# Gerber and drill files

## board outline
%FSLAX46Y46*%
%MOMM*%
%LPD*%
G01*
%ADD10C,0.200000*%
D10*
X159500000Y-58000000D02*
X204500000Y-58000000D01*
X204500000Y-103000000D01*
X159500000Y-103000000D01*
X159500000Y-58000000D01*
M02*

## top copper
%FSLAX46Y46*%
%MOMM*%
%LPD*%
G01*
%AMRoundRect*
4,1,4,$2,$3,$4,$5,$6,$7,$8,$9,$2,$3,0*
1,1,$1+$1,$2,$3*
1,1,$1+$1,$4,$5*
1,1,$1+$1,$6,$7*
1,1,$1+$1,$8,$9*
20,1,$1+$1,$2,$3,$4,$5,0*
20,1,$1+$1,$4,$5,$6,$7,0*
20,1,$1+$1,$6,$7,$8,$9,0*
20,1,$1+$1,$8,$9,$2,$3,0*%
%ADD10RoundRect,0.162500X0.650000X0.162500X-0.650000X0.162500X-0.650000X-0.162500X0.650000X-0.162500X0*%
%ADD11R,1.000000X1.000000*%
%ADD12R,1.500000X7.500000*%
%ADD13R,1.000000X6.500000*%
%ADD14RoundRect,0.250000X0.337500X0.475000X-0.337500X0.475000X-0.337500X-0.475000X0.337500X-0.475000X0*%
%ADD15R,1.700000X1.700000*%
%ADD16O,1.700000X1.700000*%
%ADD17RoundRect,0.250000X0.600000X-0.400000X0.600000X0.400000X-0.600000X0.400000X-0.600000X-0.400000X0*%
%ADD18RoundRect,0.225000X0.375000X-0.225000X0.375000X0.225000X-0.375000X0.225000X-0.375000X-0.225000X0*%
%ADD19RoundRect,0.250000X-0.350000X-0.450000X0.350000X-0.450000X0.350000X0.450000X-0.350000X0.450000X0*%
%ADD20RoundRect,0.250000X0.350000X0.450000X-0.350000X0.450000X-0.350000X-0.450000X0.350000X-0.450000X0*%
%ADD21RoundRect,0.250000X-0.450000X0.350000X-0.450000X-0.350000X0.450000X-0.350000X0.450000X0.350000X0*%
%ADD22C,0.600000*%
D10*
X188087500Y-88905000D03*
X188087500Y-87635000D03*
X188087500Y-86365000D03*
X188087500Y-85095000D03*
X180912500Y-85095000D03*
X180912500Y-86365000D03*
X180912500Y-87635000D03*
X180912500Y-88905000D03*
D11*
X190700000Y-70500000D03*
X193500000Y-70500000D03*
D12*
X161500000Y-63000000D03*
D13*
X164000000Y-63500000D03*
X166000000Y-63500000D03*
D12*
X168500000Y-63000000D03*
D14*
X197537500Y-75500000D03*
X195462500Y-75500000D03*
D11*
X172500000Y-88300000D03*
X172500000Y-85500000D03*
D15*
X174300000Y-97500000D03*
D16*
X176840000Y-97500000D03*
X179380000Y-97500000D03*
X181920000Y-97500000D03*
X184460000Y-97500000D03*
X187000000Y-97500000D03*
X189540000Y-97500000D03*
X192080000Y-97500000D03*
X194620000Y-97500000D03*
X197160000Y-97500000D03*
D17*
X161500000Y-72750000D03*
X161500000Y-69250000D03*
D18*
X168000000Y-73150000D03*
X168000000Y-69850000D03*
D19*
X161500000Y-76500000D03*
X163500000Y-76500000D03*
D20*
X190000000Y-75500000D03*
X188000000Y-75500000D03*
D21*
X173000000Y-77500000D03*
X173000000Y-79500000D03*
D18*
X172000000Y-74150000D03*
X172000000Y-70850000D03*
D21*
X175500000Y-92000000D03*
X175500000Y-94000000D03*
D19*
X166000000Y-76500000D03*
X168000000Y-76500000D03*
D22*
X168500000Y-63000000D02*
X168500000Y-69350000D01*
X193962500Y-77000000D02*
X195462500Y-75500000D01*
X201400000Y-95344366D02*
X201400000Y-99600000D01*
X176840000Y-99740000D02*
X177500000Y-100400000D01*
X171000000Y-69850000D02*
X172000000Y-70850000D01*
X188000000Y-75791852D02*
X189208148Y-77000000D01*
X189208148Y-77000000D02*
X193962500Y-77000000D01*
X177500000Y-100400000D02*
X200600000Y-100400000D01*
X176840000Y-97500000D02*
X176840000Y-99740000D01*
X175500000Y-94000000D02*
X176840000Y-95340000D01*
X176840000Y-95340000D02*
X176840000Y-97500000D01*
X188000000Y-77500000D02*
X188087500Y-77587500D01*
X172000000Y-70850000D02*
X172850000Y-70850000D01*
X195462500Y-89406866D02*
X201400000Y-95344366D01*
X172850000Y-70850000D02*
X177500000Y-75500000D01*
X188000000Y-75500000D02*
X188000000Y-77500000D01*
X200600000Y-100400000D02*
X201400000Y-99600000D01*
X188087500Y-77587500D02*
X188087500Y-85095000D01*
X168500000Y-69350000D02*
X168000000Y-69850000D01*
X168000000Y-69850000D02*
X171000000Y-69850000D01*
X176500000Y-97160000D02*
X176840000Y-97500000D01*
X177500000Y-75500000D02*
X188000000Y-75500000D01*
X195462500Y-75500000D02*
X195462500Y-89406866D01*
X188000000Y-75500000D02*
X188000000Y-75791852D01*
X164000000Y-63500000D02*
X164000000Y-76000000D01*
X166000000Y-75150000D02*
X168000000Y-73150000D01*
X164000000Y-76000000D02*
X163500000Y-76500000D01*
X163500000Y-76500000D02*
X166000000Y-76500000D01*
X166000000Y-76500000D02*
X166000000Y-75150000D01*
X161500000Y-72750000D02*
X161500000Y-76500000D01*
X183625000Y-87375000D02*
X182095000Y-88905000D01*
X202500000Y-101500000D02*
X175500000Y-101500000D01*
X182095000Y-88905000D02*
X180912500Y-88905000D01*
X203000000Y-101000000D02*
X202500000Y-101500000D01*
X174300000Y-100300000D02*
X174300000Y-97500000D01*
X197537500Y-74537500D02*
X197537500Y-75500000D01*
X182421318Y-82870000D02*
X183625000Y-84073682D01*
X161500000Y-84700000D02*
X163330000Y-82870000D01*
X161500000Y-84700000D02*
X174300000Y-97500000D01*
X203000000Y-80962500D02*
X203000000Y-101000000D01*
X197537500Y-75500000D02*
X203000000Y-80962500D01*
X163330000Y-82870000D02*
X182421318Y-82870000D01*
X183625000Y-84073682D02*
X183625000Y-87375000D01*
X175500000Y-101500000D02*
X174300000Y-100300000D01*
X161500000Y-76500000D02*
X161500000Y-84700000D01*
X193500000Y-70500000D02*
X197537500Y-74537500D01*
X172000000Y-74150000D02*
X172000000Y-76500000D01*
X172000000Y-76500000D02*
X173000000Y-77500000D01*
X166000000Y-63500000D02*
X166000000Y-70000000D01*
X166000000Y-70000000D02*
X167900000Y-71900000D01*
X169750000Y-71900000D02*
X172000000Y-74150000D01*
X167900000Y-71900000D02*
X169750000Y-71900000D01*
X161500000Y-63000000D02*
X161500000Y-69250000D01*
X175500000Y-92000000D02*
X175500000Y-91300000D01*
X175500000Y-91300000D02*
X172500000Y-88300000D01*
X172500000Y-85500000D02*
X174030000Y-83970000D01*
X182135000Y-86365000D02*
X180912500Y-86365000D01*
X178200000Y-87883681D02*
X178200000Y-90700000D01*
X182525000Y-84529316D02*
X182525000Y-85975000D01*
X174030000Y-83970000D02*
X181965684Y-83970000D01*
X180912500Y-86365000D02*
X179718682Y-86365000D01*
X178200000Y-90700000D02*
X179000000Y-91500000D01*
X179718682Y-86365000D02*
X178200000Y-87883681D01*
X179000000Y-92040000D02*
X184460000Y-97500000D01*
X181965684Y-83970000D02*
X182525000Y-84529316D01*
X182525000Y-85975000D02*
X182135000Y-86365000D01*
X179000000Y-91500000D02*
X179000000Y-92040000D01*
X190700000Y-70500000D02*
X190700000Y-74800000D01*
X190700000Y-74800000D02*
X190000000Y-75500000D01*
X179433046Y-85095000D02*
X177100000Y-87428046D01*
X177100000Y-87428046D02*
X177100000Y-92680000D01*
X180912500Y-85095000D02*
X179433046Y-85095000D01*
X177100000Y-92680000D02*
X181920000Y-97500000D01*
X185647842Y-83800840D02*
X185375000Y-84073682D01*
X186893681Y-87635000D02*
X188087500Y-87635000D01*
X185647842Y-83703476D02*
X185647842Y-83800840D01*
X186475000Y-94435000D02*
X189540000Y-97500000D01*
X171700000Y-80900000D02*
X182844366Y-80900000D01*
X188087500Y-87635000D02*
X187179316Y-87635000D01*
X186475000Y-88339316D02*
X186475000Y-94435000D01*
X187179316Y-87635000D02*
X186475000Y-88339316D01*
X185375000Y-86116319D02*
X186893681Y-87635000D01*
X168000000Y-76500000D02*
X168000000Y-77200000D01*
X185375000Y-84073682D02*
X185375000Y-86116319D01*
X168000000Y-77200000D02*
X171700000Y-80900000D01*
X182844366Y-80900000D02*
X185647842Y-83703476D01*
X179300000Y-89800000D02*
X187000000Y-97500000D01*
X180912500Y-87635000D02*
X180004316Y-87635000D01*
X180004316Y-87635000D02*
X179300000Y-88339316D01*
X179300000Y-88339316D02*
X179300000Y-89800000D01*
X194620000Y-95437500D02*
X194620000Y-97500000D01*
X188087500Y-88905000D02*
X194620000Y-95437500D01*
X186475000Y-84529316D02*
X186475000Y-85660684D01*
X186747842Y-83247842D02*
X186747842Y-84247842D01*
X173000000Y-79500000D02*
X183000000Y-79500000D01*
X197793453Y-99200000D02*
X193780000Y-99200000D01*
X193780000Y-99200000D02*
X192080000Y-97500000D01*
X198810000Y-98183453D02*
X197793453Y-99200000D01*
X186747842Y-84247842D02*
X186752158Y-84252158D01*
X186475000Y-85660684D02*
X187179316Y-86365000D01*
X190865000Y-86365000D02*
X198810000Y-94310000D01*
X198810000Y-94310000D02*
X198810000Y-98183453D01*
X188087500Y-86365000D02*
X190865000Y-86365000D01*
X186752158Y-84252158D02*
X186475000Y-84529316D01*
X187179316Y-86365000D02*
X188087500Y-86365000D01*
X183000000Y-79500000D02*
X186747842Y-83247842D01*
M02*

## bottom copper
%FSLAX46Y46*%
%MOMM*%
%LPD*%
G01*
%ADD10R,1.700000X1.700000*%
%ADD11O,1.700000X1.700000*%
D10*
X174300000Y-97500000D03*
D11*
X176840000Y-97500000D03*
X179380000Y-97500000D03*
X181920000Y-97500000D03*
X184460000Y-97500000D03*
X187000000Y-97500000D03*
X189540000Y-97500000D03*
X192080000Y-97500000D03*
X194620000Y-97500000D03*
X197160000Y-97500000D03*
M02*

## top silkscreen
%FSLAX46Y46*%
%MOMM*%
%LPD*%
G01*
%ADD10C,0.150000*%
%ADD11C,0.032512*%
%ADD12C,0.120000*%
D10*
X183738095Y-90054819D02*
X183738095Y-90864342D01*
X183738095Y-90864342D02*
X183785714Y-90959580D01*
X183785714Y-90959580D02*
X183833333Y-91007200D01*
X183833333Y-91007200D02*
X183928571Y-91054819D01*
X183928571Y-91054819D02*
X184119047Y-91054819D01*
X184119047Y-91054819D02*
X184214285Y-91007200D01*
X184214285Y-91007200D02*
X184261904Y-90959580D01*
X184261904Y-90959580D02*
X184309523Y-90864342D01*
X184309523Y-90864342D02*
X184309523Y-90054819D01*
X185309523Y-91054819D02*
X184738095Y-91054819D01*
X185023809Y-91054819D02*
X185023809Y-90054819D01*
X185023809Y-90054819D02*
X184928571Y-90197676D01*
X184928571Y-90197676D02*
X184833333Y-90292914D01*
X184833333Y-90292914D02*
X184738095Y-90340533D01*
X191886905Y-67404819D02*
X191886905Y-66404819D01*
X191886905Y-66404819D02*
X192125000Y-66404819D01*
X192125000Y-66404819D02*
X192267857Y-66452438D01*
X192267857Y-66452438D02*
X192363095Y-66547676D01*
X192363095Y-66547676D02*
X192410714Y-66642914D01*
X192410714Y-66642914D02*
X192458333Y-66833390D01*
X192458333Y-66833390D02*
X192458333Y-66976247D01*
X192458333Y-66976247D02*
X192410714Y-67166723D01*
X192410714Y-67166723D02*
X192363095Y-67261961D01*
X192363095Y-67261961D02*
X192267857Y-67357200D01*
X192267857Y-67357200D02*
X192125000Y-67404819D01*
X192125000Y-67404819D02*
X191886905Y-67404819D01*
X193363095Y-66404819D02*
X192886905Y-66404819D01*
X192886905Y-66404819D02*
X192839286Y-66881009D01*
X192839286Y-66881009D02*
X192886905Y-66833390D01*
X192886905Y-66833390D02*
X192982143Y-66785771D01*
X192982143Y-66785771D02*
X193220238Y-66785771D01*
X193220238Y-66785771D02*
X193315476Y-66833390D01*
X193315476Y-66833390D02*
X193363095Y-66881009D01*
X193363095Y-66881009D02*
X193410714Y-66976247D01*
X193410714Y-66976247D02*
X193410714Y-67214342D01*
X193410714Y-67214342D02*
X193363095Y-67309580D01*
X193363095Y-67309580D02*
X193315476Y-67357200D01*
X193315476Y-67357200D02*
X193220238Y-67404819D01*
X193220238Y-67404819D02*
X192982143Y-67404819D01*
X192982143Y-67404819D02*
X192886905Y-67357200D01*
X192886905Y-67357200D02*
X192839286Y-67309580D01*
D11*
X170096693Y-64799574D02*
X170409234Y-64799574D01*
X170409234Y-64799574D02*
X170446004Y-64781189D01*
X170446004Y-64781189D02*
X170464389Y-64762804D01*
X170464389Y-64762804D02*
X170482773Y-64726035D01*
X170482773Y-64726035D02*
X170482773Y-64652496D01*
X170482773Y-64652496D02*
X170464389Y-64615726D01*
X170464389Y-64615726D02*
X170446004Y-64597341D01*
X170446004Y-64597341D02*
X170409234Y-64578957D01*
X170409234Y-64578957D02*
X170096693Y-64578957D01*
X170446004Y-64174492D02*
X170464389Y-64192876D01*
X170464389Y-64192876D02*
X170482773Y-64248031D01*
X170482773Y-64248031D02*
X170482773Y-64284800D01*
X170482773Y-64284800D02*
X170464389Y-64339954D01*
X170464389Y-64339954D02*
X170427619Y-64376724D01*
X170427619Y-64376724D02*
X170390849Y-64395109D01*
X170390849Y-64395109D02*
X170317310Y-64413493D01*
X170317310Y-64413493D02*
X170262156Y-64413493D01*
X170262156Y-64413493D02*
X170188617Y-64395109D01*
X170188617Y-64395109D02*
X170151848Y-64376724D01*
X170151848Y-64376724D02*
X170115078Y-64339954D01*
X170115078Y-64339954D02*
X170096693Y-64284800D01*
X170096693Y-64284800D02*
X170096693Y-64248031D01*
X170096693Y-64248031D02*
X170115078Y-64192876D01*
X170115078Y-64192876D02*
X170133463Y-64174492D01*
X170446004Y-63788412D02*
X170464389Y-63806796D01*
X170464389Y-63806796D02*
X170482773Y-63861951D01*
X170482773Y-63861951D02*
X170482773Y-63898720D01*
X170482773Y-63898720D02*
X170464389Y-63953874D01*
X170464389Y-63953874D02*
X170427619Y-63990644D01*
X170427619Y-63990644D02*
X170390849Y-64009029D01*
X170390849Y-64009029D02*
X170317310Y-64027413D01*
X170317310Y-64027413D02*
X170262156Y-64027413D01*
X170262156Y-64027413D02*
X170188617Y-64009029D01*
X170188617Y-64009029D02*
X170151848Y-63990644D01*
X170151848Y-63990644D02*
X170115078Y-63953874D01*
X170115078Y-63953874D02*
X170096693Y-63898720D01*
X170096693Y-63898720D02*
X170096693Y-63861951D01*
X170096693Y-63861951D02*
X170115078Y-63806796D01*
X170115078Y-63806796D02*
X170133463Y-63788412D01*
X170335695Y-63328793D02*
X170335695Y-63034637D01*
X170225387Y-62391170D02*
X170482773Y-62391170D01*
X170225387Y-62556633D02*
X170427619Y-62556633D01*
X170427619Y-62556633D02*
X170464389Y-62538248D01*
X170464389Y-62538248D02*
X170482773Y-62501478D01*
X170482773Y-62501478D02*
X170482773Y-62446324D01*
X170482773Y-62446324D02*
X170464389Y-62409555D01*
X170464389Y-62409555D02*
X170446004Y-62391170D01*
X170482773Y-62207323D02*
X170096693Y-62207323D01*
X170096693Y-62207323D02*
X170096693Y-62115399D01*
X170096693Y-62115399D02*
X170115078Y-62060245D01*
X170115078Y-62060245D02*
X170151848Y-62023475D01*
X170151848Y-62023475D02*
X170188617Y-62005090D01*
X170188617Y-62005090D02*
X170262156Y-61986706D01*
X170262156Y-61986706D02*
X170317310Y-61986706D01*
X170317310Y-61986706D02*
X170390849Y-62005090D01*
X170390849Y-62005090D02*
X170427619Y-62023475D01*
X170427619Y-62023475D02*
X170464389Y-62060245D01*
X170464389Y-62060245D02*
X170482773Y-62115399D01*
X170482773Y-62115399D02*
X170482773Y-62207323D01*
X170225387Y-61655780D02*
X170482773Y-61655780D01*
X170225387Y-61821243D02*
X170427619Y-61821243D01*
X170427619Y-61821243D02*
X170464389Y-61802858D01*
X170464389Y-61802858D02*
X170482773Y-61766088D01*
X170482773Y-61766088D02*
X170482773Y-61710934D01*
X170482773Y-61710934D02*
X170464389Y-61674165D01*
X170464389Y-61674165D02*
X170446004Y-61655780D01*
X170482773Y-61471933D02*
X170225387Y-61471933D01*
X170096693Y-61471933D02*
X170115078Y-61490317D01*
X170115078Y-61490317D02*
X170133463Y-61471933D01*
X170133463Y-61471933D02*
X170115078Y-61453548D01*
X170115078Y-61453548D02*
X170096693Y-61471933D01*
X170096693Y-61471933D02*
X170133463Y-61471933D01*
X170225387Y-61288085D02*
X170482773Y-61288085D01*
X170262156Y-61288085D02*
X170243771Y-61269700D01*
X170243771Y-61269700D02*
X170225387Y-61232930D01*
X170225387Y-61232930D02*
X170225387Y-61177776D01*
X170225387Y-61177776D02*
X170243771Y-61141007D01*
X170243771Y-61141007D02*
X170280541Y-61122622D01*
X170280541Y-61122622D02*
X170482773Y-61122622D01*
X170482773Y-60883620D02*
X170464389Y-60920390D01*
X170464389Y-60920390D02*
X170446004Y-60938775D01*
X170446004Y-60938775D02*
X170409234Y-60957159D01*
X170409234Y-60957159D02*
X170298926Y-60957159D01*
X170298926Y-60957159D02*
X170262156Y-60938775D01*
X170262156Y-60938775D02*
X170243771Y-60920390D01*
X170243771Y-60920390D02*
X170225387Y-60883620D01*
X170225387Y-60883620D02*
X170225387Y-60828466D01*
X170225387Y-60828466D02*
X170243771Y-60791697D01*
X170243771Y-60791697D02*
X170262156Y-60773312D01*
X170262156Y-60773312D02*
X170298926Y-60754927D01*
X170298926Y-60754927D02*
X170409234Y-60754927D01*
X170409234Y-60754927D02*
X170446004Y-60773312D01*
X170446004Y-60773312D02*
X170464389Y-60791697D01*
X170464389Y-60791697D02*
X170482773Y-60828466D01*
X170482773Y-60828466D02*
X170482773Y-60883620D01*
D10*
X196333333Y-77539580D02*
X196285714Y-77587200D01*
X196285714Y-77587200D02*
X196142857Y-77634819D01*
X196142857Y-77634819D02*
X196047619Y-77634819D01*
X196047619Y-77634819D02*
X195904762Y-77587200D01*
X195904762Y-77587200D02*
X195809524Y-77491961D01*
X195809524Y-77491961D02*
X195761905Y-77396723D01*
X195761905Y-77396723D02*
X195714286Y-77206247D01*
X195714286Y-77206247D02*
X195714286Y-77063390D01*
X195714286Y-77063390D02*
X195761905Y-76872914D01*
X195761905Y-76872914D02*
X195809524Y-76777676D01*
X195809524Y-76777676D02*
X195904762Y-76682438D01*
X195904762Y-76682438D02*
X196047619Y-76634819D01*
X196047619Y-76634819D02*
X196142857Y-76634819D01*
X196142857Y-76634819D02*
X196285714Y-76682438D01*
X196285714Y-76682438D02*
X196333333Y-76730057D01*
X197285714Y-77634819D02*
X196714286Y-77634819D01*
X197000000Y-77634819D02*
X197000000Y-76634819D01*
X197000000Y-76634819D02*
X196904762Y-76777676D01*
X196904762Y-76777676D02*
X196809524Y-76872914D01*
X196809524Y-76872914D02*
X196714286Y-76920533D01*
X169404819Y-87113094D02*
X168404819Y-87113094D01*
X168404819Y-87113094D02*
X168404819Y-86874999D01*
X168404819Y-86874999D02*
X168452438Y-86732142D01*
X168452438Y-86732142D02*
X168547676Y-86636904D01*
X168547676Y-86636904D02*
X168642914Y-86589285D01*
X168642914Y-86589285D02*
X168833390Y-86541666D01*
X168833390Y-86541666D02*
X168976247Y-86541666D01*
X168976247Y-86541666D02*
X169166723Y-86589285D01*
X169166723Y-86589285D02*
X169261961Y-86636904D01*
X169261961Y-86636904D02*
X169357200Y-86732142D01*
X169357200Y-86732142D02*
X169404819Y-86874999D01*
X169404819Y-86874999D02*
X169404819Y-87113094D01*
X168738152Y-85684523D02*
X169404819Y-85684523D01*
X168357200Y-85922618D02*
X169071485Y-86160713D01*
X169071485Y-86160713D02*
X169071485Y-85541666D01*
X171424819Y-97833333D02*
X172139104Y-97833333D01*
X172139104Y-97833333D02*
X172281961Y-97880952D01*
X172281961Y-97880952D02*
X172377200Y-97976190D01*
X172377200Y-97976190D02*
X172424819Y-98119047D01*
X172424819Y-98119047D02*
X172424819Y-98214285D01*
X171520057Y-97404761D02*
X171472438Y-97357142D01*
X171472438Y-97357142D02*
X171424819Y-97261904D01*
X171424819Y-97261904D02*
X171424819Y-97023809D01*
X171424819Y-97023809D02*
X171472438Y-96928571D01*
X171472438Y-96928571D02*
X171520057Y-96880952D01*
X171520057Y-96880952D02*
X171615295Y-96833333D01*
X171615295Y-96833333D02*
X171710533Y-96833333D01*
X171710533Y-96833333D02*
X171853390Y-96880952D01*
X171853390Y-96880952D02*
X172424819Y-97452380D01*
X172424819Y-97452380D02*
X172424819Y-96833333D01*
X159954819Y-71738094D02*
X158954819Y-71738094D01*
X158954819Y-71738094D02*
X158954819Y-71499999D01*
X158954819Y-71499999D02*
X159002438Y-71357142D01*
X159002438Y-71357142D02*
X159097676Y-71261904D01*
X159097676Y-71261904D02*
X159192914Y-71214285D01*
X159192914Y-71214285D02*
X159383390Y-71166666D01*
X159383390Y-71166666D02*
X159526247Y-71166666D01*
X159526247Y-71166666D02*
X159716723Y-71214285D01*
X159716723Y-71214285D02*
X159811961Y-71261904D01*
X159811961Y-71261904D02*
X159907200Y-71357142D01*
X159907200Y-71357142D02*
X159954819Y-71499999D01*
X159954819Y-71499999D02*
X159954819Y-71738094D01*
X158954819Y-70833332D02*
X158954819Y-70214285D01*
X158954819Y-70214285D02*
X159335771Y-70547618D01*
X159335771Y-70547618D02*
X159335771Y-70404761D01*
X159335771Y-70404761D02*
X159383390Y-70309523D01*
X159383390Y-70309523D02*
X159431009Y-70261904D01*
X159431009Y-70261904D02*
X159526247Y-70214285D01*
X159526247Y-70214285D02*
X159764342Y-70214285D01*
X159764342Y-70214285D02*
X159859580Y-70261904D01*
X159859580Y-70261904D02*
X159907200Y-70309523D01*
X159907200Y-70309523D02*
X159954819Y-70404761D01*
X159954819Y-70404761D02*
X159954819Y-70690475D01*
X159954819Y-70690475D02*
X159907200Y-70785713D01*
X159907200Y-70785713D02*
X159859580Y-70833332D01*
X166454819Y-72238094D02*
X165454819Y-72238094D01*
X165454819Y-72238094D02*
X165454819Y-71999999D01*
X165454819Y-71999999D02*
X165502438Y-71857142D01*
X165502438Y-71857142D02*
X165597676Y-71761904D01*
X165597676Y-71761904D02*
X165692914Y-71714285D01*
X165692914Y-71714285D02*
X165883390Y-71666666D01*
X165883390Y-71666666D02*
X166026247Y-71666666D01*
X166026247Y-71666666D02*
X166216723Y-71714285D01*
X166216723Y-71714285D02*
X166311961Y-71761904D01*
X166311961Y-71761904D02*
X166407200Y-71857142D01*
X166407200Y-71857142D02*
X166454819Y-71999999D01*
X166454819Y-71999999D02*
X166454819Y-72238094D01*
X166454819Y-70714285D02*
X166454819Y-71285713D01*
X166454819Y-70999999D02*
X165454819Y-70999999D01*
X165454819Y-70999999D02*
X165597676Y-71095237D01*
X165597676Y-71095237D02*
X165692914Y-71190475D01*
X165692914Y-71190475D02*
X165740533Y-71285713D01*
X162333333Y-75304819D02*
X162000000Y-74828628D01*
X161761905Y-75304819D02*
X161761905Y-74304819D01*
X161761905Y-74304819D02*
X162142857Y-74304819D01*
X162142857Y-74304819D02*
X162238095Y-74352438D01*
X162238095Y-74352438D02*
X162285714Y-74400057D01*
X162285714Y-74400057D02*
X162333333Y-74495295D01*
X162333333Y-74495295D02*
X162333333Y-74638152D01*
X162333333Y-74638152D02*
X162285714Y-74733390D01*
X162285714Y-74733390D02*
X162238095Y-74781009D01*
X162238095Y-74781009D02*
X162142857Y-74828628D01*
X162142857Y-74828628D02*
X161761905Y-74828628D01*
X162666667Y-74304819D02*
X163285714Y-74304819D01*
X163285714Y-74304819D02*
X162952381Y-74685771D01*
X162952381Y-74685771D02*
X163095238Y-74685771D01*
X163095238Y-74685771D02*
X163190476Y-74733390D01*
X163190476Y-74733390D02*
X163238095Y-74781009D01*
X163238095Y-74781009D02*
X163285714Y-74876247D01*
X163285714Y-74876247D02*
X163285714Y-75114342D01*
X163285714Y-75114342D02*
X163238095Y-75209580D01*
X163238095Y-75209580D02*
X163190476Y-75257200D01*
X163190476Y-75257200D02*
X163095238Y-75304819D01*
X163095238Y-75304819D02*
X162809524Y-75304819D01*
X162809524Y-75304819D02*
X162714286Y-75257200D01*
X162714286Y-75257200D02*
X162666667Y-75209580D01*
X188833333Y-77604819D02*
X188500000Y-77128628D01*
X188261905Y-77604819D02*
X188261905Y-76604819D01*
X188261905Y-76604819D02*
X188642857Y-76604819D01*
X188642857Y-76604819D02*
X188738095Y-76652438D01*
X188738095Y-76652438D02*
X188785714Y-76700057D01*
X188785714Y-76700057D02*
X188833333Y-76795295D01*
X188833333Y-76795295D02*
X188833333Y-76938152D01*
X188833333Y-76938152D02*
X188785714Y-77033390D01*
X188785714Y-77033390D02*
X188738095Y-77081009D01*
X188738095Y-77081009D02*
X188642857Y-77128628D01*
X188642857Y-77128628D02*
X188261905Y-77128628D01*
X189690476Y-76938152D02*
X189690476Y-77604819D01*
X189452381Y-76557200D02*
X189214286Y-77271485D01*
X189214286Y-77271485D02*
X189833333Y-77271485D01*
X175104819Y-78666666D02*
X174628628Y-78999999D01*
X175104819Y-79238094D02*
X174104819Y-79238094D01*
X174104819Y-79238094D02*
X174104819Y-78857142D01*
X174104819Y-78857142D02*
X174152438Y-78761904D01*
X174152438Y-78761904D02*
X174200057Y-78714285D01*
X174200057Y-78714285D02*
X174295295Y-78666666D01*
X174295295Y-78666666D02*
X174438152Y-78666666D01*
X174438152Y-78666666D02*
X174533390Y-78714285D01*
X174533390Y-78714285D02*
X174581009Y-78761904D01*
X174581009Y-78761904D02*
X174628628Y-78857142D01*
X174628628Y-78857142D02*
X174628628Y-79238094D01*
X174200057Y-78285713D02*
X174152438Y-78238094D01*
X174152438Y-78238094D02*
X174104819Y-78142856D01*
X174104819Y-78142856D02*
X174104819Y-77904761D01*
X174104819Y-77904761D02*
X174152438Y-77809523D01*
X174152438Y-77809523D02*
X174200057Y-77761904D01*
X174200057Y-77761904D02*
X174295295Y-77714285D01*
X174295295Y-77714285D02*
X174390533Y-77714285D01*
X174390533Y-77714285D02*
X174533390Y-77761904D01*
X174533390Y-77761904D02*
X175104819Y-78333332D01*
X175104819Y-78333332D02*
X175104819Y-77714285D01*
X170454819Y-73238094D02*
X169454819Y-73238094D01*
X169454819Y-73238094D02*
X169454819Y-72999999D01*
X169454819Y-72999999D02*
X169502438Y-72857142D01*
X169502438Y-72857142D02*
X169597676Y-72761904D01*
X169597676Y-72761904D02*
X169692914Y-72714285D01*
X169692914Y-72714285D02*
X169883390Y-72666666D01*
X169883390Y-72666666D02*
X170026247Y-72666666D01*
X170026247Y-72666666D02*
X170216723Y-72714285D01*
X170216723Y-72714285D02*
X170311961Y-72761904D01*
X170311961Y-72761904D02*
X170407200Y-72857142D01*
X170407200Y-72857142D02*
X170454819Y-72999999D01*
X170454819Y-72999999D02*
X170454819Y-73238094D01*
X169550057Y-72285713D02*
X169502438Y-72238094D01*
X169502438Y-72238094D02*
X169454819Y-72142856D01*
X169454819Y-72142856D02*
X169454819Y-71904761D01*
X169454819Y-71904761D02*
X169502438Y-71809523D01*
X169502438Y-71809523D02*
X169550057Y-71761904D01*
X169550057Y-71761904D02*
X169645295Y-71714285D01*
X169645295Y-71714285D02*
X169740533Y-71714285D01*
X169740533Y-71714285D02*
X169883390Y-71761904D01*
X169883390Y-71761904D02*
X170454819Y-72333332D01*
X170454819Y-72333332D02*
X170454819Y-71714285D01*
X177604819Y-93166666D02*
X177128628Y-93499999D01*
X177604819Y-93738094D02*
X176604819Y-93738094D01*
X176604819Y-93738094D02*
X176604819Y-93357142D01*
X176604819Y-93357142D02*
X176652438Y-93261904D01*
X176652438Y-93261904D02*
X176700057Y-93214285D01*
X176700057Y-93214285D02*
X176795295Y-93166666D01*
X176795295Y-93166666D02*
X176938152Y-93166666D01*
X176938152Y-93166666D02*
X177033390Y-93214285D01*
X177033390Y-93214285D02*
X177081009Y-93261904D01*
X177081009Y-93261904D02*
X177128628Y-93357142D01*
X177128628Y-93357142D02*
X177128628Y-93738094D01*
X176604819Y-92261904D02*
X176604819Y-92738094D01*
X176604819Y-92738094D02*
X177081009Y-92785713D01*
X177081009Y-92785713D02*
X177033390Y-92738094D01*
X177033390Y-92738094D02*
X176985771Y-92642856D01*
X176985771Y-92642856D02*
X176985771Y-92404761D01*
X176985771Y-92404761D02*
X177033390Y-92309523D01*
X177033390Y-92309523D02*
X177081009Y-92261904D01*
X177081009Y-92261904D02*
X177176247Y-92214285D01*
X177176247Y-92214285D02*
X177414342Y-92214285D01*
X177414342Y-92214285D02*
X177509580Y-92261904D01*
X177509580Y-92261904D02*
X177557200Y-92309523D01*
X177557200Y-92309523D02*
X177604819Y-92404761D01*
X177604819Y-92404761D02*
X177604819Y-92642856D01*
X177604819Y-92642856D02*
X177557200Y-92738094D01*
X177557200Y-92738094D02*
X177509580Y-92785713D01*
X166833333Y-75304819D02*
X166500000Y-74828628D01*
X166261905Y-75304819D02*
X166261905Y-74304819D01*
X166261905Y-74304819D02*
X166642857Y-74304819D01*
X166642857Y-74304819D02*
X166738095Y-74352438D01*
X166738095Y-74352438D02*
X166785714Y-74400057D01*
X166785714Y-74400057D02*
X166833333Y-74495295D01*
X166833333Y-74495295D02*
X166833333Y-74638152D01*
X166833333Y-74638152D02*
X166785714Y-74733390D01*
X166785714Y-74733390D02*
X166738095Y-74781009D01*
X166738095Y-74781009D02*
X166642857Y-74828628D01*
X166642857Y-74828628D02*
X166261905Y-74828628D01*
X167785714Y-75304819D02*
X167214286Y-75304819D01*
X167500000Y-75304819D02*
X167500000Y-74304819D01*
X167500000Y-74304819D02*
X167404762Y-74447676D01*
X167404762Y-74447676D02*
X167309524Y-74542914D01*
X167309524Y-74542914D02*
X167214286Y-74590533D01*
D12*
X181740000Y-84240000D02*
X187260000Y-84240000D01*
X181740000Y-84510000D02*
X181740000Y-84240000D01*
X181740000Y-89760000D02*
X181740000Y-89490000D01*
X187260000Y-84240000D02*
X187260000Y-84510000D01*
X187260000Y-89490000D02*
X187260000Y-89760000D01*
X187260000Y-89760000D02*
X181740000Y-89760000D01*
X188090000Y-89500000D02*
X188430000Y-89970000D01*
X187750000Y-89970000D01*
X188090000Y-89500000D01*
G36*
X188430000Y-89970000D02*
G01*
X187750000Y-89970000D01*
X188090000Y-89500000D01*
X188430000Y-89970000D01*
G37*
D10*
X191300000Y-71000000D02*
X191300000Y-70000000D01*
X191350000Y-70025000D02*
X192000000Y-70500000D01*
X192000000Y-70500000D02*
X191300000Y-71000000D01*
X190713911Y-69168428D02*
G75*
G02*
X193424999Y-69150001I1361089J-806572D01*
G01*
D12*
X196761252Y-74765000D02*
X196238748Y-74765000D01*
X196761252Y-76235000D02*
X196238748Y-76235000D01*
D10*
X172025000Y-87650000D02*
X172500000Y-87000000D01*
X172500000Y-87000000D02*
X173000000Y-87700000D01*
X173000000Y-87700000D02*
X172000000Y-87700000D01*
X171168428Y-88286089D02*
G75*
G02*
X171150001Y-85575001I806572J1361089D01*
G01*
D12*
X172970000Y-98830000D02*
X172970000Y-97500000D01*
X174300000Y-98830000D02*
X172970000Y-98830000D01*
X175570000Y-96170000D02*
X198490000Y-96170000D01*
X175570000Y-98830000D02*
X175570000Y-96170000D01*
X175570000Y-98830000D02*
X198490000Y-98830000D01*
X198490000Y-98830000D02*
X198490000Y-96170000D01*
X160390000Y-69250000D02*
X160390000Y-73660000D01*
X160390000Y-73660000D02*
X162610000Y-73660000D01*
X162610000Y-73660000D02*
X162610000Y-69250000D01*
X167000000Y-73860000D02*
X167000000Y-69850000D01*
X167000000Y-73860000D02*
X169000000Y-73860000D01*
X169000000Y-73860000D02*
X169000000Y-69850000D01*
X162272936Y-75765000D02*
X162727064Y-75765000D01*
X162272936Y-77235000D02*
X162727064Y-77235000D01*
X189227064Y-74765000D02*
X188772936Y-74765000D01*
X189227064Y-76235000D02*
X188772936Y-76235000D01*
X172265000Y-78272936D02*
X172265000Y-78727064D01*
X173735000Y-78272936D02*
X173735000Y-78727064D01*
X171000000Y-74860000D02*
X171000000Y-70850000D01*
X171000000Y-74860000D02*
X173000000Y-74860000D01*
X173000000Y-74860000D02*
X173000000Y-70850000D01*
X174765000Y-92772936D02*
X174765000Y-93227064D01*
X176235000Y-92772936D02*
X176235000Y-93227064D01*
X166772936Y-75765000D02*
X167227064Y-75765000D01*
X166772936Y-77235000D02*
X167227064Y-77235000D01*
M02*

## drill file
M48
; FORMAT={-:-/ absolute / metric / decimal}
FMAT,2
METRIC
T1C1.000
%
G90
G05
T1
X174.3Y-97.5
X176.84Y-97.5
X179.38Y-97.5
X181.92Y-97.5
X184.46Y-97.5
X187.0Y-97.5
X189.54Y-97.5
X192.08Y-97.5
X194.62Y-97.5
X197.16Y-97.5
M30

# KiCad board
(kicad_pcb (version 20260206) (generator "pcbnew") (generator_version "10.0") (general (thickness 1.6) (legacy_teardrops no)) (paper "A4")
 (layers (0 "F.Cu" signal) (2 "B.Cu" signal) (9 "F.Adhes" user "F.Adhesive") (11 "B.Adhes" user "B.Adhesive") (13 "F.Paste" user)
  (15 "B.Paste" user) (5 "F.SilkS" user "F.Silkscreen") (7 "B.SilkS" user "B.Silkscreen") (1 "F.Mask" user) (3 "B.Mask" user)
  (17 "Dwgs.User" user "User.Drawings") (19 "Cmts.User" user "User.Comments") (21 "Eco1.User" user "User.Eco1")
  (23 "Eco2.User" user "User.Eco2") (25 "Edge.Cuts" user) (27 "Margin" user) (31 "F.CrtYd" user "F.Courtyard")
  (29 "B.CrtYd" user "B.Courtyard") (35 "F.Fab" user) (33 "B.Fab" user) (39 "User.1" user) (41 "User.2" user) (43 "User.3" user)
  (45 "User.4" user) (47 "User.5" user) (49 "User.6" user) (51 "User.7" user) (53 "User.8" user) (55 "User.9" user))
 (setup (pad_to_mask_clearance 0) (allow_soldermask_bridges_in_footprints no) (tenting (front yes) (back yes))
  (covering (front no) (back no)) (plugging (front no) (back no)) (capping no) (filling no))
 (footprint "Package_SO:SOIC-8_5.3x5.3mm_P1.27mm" (layer "F.Cu") (at 184.5 87 180)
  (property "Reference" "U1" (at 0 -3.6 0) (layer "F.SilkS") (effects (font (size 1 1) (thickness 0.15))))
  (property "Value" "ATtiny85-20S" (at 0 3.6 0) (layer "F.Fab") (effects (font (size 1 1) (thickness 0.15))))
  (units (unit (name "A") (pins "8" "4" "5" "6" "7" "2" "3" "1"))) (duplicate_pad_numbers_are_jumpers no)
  (fp_line (start 2.76 2.76) (end -2.76 2.76) (stroke (width 0.12) (type solid)) (layer "F.SilkS"))
  (fp_line (start 2.76 2.49) (end 2.76 2.76) (stroke (width 0.12) (type solid)) (layer "F.SilkS"))
  (fp_line (start 2.76 -2.76) (end 2.76 -2.49) (stroke (width 0.12) (type solid)) (layer "F.SilkS"))
  (fp_line (start -2.76 2.76) (end -2.76 2.49) (stroke (width 0.12) (type solid)) (layer "F.SilkS"))
  (fp_line (start -2.76 -2.49) (end -2.76 -2.76) (stroke (width 0.12) (type solid)) (layer "F.SilkS"))
  (fp_line (start -2.76 -2.76) (end 2.76 -2.76) (stroke (width 0.12) (type solid)) (layer "F.SilkS"))
  (fp_poly (pts (xy -3.59 -2.5) (xy -3.93 -2.97) (xy -3.25 -2.97)) (stroke (width 0.12) (type solid)) (fill yes) (layer "F.SilkS"))
  (pad "1" smd roundrect (at -3.5875 -1.905 180) (size 1.625 0.65) (layers "F.Cu" "F.Mask" "F.Paste") (roundrect_rratio 0.25)
   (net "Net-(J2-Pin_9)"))
  (pad "2" smd roundrect (at -3.5875 -0.635 180) (size 1.625 0.65) (layers "F.Cu" "F.Mask" "F.Paste") (roundrect_rratio 0.25)
   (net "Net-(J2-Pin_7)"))
  (pad "3" smd roundrect (at -3.5875 0.635 180) (size 1.625 0.65) (layers "F.Cu" "F.Mask" "F.Paste") (roundrect_rratio 0.25)
   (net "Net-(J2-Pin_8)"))
  (pad "4" smd roundrect (at -3.5875 1.905 180) (size 1.625 0.65) (layers "F.Cu" "F.Mask" "F.Paste") (roundrect_rratio 0.25) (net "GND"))
  (pad "5" smd roundrect (at 3.5875 1.905 180) (size 1.625 0.65) (layers "F.Cu" "F.Mask" "F.Paste") (roundrect_rratio 0.25)
   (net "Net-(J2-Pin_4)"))
  (pad "6" smd roundrect (at 3.5875 0.635 180) (size 1.625 0.65) (layers "F.Cu" "F.Mask" "F.Paste") (roundrect_rratio 0.25)
   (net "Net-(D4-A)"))
  (pad "7" smd roundrect (at 3.5875 -0.635 180) (size 1.625 0.65) (layers "F.Cu" "F.Mask" "F.Paste") (roundrect_rratio 0.25)
   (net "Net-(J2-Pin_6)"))
  (pad "8" smd roundrect (at 3.5875 -1.905 180) (size 1.625 0.65) (layers "F.Cu" "F.Mask" "F.Paste") (roundrect_rratio 0.25) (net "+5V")))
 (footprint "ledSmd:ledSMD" (layer "F.Cu") (at 192.5 70.5)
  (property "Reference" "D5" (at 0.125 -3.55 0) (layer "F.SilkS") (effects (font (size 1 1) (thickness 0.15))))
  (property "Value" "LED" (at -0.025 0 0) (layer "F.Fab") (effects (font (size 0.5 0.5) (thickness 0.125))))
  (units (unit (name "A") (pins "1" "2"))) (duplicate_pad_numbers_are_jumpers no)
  (fp_line (start -1.2 0.5) (end -1.2 -0.5) (stroke (width 0.15) (type solid)) (layer "F.SilkS"))
  (fp_line (start -1.15 -0.475) (end -0.5 0) (stroke (width 0.15) (type solid)) (layer "F.SilkS"))
  (fp_line (start -0.5 0) (end -1.2 0.5) (stroke (width 0.15) (type solid)) (layer "F.SilkS"))
  (fp_arc (start -1.786089 -1.331572) (mid -0.435753 -2.107089) (end 0.924999 -1.349999) (stroke (width 0.15) (type solid))
   (layer "F.SilkS"))
  (pad "1" smd rect (at -1.8 0) (size 1 1) (layers "F.Cu" "F.Mask" "F.Paste") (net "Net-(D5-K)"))
  (pad "2" smd rect (at 1 0) (size 1 1) (layers "F.Cu" "F.Mask" "F.Paste") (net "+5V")))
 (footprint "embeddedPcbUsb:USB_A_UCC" (layer "F.Cu") (at 165 63.2 -90)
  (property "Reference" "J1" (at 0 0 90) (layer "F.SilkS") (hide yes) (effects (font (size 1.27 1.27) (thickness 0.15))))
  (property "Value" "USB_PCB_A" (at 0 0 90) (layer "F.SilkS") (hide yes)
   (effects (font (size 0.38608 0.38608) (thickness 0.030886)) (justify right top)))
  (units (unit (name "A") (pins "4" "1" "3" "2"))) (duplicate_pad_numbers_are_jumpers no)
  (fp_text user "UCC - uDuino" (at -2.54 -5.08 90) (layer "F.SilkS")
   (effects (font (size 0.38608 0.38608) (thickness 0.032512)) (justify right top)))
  (pad "1" smd rect (at -0.2 3.5 270) (size 7.5 1.5) (layers "F.Cu" "F.Mask" "F.Paste") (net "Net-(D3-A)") (solder_mask_margin 0.1016))
  (pad "2" smd rect (at 0.3 1 270) (size 6.5 1) (layers "F.Cu" "F.Mask" "F.Paste") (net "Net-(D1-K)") (solder_mask_margin 0.1016))
  (pad "3" smd rect (at 0.3 -1 270) (size 6.5 1) (layers "F.Cu" "F.Mask" "F.Paste") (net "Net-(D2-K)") (solder_mask_margin 0.1016))
  (pad "4" smd rect (at -0.2 -3.5 270) (size 7.5 1.5) (layers "F.Cu" "F.Mask" "F.Paste") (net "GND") (solder_mask_margin 0.1016)))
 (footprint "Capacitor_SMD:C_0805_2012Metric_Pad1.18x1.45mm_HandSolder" (layer "F.Cu") (at 196.5 75.5 180)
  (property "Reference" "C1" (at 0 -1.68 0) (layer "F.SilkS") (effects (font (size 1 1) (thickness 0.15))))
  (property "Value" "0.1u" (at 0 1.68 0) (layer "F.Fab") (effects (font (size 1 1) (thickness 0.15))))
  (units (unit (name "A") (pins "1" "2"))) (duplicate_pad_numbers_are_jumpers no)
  (fp_line (start -0.261252 0.735) (end 0.261252 0.735) (stroke (width 0.12) (type solid)) (layer "F.SilkS"))
  (fp_line (start -0.261252 -0.735) (end 0.261252 -0.735) (stroke (width 0.12) (type solid)) (layer "F.SilkS"))
  (pad "1" smd roundrect (at -1.0375 0 180) (size 1.175 1.45) (layers "F.Cu" "F.Mask" "F.Paste") (roundrect_rratio 0.212766) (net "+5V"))
  (pad "2" smd roundrect (at 1.0375 0 180) (size 1.175 1.45) (layers "F.Cu" "F.Mask" "F.Paste") (roundrect_rratio 0.212766) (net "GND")))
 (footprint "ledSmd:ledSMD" (layer "F.Cu") (at 172.5 86.5 90)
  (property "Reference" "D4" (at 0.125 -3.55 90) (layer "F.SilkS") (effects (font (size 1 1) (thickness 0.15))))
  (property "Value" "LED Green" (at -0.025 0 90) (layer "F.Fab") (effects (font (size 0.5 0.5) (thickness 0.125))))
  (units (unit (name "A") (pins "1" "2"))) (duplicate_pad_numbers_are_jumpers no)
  (fp_line (start -1.15 -0.475) (end -0.5 0) (stroke (width 0.15) (type solid)) (layer "F.SilkS"))
  (fp_line (start -0.5 0) (end -1.2 0.5) (stroke (width 0.15) (type solid)) (layer "F.SilkS"))
  (fp_line (start -1.2 0.5) (end -1.2 -0.5) (stroke (width 0.15) (type solid)) (layer "F.SilkS"))
  (fp_arc (start -1.786089 -1.331572) (mid -0.435753 -2.107089) (end 0.924999 -1.349999) (stroke (width 0.15) (type solid))
   (layer "F.SilkS"))
  (pad "1" smd rect (at -1.8 0 90) (size 1 1) (layers "F.Cu" "F.Mask" "F.Paste") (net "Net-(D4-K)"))
  (pad "2" smd rect (at 1 0 90) (size 1 1) (layers "F.Cu" "F.Mask" "F.Paste") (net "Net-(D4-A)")))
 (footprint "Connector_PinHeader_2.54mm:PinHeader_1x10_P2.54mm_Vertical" (layer "F.Cu") (at 174.3 97.5 90)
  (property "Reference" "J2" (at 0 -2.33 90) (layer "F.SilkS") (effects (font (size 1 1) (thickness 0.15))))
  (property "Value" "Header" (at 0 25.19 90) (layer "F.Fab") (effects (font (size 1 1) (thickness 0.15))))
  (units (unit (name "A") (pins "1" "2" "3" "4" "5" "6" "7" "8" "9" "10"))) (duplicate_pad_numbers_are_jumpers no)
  (fp_line (start -1.33 -1.33) (end 0 -1.33) (stroke (width 0.12) (type solid)) (layer "F.SilkS"))
  (fp_line (start -1.33 0) (end -1.33 -1.33) (stroke (width 0.12) (type solid)) (layer "F.SilkS"))
  (fp_line (start 1.33 1.27) (end 1.33 24.19) (stroke (width 0.12) (type solid)) (layer "F.SilkS"))
  (fp_line (start -1.33 1.27) (end 1.33 1.27) (stroke (width 0.12) (type solid)) (layer "F.SilkS"))
  (fp_line (start -1.33 1.27) (end -1.33 24.19) (stroke (width 0.12) (type solid)) (layer "F.SilkS"))
  (fp_line (start -1.33 24.19) (end 1.33 24.19) (stroke (width 0.12) (type solid)) (layer "F.SilkS"))
  (pad "1" thru_hole rect (at 0 0 90) (size 1.7 1.7) (drill 1) (layers "*.Cu" "*.Mask") (remove_unused_layers no) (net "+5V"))
  (pad "2" thru_hole oval (at 0 2.54 90) (size 1.7 1.7) (drill 1) (layers "*.Cu" "*.Mask") (remove_unused_layers no) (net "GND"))
  (pad "3" thru_hole oval (at 0 5.08 90) (size 1.7 1.7) (drill 1) (layers "*.Cu" "*.Mask") (remove_unused_layers no)
   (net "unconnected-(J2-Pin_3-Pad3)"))
  (pad "4" thru_hole oval (at 0 7.62 90) (size 1.7 1.7) (drill 1) (layers "*.Cu" "*.Mask") (remove_unused_layers no) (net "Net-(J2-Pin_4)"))
  (pad "5" thru_hole oval (at 0 10.16 90) (size 1.7 1.7) (drill 1) (layers "*.Cu" "*.Mask") (remove_unused_layers no) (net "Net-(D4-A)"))
  (pad "6" thru_hole oval (at 0 12.7 90) (size 1.7 1.7) (drill 1) (layers "*.Cu" "*.Mask") (remove_unused_layers no) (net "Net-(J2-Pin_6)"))
  (pad "7" thru_hole oval (at 0 15.24 90) (size 1.7 1.7) (drill 1) (layers "*.Cu" "*.Mask") (remove_unused_layers no) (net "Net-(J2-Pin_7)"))
  (pad "8" thru_hole oval (at 0 17.78 90) (size 1.7 1.7) (drill 1) (layers "*.Cu" "*.Mask") (remove_unused_layers no) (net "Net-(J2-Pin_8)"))
  (pad "9" thru_hole oval (at 0 20.32 90) (size 1.7 1.7) (drill 1) (layers "*.Cu" "*.Mask") (remove_unused_layers no) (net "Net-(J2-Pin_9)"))
  (pad "10" thru_hole oval (at 0 22.86 90) (size 1.7 1.7) (drill 1) (layers "*.Cu" "*.Mask") (remove_unused_layers no)
   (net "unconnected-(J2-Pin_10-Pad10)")))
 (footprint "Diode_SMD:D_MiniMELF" (layer "F.Cu") (at 161.5 71 90)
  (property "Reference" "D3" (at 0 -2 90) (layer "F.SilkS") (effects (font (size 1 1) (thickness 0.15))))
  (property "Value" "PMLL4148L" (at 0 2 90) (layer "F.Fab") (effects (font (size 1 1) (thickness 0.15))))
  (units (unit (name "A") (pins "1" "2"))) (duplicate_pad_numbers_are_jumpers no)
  (fp_line (start 1.75 -1.11) (end -2.66 -1.11) (stroke (width 0.12) (type solid)) (layer "F.SilkS"))
  (fp_line (start -2.66 -1.11) (end -2.66 1.11) (stroke (width 0.12) (type solid)) (layer "F.SilkS"))
  (fp_line (start -2.66 1.11) (end 1.75 1.11) (stroke (width 0.12) (type solid)) (layer "F.SilkS"))
  (pad "1" smd roundrect (at -1.75 0 90) (size 1.3 1.7) (layers "F.Cu" "F.Mask" "F.Paste") (roundrect_rratio 0.1923076923) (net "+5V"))
  (pad "2" smd roundrect (at 1.75 0 90) (size 1.3 1.7) (layers "F.Cu" "F.Mask" "F.Paste") (roundrect_rratio 0.1923076923) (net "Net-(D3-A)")))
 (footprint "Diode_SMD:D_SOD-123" (layer "F.Cu") (at 168 71.5 90)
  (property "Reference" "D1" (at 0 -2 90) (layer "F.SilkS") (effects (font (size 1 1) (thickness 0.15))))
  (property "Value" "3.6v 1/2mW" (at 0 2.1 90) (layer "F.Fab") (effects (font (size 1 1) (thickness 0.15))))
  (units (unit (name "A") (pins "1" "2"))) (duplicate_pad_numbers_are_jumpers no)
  (fp_line (start -2.36 -1) (end 1.65 -1) (stroke (width 0.12) (type solid)) (layer "F.SilkS"))
  (fp_line (start -2.36 -1) (end -2.36 1) (stroke (width 0.12) (type solid)) (layer "F.SilkS"))
  (fp_line (start -2.36 1) (end 1.65 1) (stroke (width 0.12) (type solid)) (layer "F.SilkS"))
  (pad "1" smd roundrect (at -1.65 0 90) (size 0.9 1.2) (layers "F.Cu" "F.Mask" "F.Paste") (roundrect_rratio 0.25) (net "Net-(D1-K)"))
  (pad "2" smd roundrect (at 1.65 0 90) (size 0.9 1.2) (layers "F.Cu" "F.Mask" "F.Paste") (roundrect_rratio 0.25) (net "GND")))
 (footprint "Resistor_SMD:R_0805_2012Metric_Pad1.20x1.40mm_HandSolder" (layer "F.Cu") (at 162.5 76.5)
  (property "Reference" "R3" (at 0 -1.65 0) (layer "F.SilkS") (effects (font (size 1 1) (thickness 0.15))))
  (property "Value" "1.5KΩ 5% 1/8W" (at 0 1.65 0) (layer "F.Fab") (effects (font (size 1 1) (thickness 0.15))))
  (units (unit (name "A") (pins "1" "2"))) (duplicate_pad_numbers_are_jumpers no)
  (fp_line (start -0.227064 -0.735) (end 0.227064 -0.735) (stroke (width 0.12) (type solid)) (layer "F.SilkS"))
  (fp_line (start -0.227064 0.735) (end 0.227064 0.735) (stroke (width 0.12) (type solid)) (layer "F.SilkS"))
  (pad "1" smd roundrect (at -1 0) (size 1.2 1.4) (layers "F.Cu" "F.Mask" "F.Paste") (roundrect_rratio 0.208333) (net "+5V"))
  (pad "2" smd roundrect (at 1 0) (size 1.2 1.4) (layers "F.Cu" "F.Mask" "F.Paste") (roundrect_rratio 0.208333) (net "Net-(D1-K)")))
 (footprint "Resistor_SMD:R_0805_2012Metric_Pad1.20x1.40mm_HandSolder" (layer "F.Cu") (at 189 75.5 180)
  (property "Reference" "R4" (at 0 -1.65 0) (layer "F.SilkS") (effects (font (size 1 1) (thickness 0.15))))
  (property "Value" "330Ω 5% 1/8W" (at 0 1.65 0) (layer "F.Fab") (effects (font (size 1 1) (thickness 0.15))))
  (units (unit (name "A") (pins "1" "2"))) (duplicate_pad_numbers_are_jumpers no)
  (fp_line (start -0.227064 0.735) (end 0.227064 0.735) (stroke (width 0.12) (type solid)) (layer "F.SilkS"))
  (fp_line (start -0.227064 -0.735) (end 0.227064 -0.735) (stroke (width 0.12) (type solid)) (layer "F.SilkS"))
  (pad "1" smd roundrect (at -1 0 180) (size 1.2 1.4) (layers "F.Cu" "F.Mask" "F.Paste") (roundrect_rratio 0.208333) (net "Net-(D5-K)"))
  (pad "2" smd roundrect (at 1 0 180) (size 1.2 1.4) (layers "F.Cu" "F.Mask" "F.Paste") (roundrect_rratio 0.208333) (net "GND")))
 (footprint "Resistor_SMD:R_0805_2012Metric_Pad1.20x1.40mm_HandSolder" (layer "F.Cu") (at 173 78.5 -90)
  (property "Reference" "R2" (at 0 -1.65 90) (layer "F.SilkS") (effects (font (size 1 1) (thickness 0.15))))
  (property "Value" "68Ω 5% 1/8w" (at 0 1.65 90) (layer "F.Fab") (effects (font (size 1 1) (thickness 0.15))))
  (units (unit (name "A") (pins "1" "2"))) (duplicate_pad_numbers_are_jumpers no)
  (fp_line (start -0.227064 0.735) (end 0.227064 0.735) (stroke (width 0.12) (type solid)) (layer "F.SilkS"))
  (fp_line (start -0.227064 -0.735) (end 0.227064 -0.735) (stroke (width 0.12) (type solid)) (layer "F.SilkS"))
  (pad "1" smd roundrect (at -1 0 270) (size 1.2 1.4) (layers "F.Cu" "F.Mask" "F.Paste") (roundrect_rratio 0.208333) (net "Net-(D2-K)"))
  (pad "2" smd roundrect (at 1 0 270) (size 1.2 1.4) (layers "F.Cu" "F.Mask" "F.Paste") (roundrect_rratio 0.208333) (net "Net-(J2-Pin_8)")))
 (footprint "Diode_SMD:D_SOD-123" (layer "F.Cu") (at 172 72.5 90)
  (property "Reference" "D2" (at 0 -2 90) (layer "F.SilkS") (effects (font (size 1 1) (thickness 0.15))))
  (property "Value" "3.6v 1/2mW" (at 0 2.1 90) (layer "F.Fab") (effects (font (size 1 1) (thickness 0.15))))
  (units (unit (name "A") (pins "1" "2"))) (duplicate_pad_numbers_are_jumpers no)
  (fp_line (start -2.36 -1) (end 1.65 -1) (stroke (width 0.12) (type solid)) (layer "F.SilkS"))
  (fp_line (start -2.36 -1) (end -2.36 1) (stroke (width 0.12) (type solid)) (layer "F.SilkS"))
  (fp_line (start -2.36 1) (end 1.65 1) (stroke (width 0.12) (type solid)) (layer "F.SilkS"))
  (pad "1" smd roundrect (at -1.65 0 90) (size 0.9 1.2) (layers "F.Cu" "F.Mask" "F.Paste") (roundrect_rratio 0.25) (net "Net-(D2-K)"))
  (pad "2" smd roundrect (at 1.65 0 90) (size 0.9 1.2) (layers "F.Cu" "F.Mask" "F.Paste") (roundrect_rratio 0.25) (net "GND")))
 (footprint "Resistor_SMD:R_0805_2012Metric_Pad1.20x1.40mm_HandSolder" (layer "F.Cu") (at 175.5 93 -90)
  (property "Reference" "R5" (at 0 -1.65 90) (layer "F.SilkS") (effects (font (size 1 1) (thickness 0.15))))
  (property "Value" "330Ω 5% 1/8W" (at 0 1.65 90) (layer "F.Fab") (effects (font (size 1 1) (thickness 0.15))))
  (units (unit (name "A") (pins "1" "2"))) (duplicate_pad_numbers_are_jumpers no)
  (fp_line (start -0.227064 0.735) (end 0.227064 0.735) (stroke (width 0.12) (type solid)) (layer "F.SilkS"))
  (fp_line (start -0.227064 -0.735) (end 0.227064 -0.735) (stroke (width 0.12) (type solid)) (layer "F.SilkS"))
  (pad "1" smd roundrect (at -1 0 270) (size 1.2 1.4) (layers "F.Cu" "F.Mask" "F.Paste") (roundrect_rratio 0.208333) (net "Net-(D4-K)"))
  (pad "2" smd roundrect (at 1 0 270) (size 1.2 1.4) (layers "F.Cu" "F.Mask" "F.Paste") (roundrect_rratio 0.208333) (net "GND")))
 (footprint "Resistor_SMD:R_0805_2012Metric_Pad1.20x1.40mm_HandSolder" (layer "F.Cu") (at 167 76.5)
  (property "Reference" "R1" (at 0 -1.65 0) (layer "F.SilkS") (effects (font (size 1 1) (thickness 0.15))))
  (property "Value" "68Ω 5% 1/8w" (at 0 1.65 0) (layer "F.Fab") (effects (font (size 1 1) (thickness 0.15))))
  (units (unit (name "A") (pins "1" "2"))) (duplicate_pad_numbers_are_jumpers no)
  (fp_line (start -0.227064 -0.735) (end 0.227064 -0.735) (stroke (width 0.12) (type solid)) (layer "F.SilkS"))
  (fp_line (start -0.227064 0.735) (end 0.227064 0.735) (stroke (width 0.12) (type solid)) (layer "F.SilkS"))
  (pad "1" smd roundrect (at -1 0) (size 1.2 1.4) (layers "F.Cu" "F.Mask" "F.Paste") (roundrect_rratio 0.208333) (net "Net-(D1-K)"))
  (pad "2" smd roundrect (at 1 0) (size 1.2 1.4) (layers "F.Cu" "F.Mask" "F.Paste") (roundrect_rratio 0.208333) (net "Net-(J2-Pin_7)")))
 (gr_rect (start 159.5 58) (end 204.5 103) (stroke (width 0.2) (type solid)) (fill no) (layer "Edge.Cuts"))
 (segment (start 168.5 63) (end 168.5 69.35) (width 0.6) (layer "F.Cu") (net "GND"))
 (segment (start 193.9625 77) (end 195.4625 75.5) (width 0.6) (layer "F.Cu") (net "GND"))
 (segment (start 201.4 95.344366) (end 201.4 99.6) (width 0.6) (layer "F.Cu") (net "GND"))
 (segment (start 176.84 99.74) (end 177.5 100.4) (width 0.6) (layer "F.Cu") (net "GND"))
 (segment (start 171 69.85) (end 172 70.85) (width 0.6) (layer "F.Cu") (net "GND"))
 (segment (start 188 75.791852) (end 189.208148 77) (width 0.6) (layer "F.Cu") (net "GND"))
 (segment (start 189.208148 77) (end 193.9625 77) (width 0.6) (layer "F.Cu") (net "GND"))
 (segment (start 177.5 100.4) (end 200.6 100.4) (width 0.6) (layer "F.Cu") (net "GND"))
 (segment (start 176.84 97.5) (end 176.84 99.74) (width 0.6) (layer "F.Cu") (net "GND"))
 (segment (start 175.5 94) (end 176.84 95.34) (width 0.6) (layer "F.Cu") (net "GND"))
 (segment (start 176.84 95.34) (end 176.84 97.5) (width 0.6) (layer "F.Cu") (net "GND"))
 (segment (start 188 77.5) (end 188.0875 77.5875) (width 0.6) (layer "F.Cu") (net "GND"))
 (segment (start 172 70.85) (end 172.85 70.85) (width 0.6) (layer "F.Cu") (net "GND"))
 (segment (start 195.4625 89.406866) (end 201.4 95.344366) (width 0.6) (layer "F.Cu") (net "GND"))
 (segment (start 172.85 70.85) (end 177.5 75.5) (width 0.6) (layer "F.Cu") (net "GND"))
 (segment (start 188 75.5) (end 188 77.5) (width 0.6) (layer "F.Cu") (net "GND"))
 (segment (start 200.6 100.4) (end 201.4 99.6) (width 0.6) (layer "F.Cu") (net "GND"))
 (segment (start 188.0875 77.5875) (end 188.0875 85.095) (width 0.6) (layer "F.Cu") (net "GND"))
 (segment (start 168.5 69.35) (end 168 69.85) (width 0.6) (layer "F.Cu") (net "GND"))
 (segment (start 168 69.85) (end 171 69.85) (width 0.6) (layer "F.Cu") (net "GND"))
 (segment (start 176.5 97.16) (end 176.84 97.5) (width 0.6) (layer "F.Cu") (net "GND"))
 (segment (start 177.5 75.5) (end 188 75.5) (width 0.6) (layer "F.Cu") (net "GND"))
 (segment (start 195.4625 75.5) (end 195.4625 89.406866) (width 0.6) (layer "F.Cu") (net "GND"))
 (segment (start 188 75.5) (end 188 75.791852) (width 0.6) (layer "F.Cu") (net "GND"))
 (segment (start 164 63.5) (end 164 76) (width 0.6) (layer "F.Cu") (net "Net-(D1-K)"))
 (segment (start 166 75.15) (end 168 73.15) (width 0.6) (layer "F.Cu") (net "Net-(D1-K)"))
 (segment (start 164 76) (end 163.5 76.5) (width 0.6) (layer "F.Cu") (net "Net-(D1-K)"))
 (segment (start 163.5 76.5) (end 166 76.5) (width 0.6) (layer "F.Cu") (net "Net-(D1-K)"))
 (segment (start 166 76.5) (end 166 75.15) (width 0.6) (layer "F.Cu") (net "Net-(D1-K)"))
 (segment (start 161.5 72.75) (end 161.5 76.5) (width 0.6) (layer "F.Cu") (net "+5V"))
 (segment (start 183.625 87.375) (end 182.095 88.905) (width 0.6) (layer "F.Cu") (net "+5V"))
 (segment (start 202.5 101.5) (end 175.5 101.5) (width 0.6) (layer "F.Cu") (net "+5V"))
 (segment (start 182.095 88.905) (end 180.9125 88.905) (width 0.6) (layer "F.Cu") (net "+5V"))
 (segment (start 203 101) (end 202.5 101.5) (width 0.6) (layer "F.Cu") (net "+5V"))
 (segment (start 174.3 100.3) (end 174.3 97.5) (width 0.6) (layer "F.Cu") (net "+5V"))
 (segment (start 197.5375 74.5375) (end 197.5375 75.5) (width 0.6) (layer "F.Cu") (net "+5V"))
 (segment (start 182.421318 82.87) (end 183.625 84.073682) (width 0.6) (layer "F.Cu") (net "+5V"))
 (segment (start 161.5 84.7) (end 163.33 82.87) (width 0.6) (layer "F.Cu") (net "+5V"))
 (segment (start 161.5 84.7) (end 174.3 97.5) (width 0.6) (layer "F.Cu") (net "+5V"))
 (segment (start 203 80.9625) (end 203 101) (width 0.6) (layer "F.Cu") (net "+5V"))
 (segment (start 197.5375 75.5) (end 203 80.9625) (width 0.6) (layer "F.Cu") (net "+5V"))
 (segment (start 163.33 82.87) (end 182.421318 82.87) (width 0.6) (layer "F.Cu") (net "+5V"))
 (segment (start 183.625 84.073682) (end 183.625 87.375) (width 0.6) (layer "F.Cu") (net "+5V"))
 (segment (start 175.5 101.5) (end 174.3 100.3) (width 0.6) (layer "F.Cu") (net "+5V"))
 (segment (start 161.5 76.5) (end 161.5 84.7) (width 0.6) (layer "F.Cu") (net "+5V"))
 (segment (start 193.5 70.5) (end 197.5375 74.5375) (width 0.6) (layer "F.Cu") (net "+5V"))
 (segment (start 172 74.15) (end 172 76.5) (width 0.6) (layer "F.Cu") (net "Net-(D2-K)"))
 (segment (start 172 76.5) (end 173 77.5) (width 0.6) (layer "F.Cu") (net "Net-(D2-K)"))
 (segment (start 166 63.5) (end 166 70) (width 0.6) (layer "F.Cu") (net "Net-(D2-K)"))
 (segment (start 166 70) (end 167.9 71.9) (width 0.6) (layer "F.Cu") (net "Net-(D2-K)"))
 (segment (start 169.75 71.9) (end 172 74.15) (width 0.6) (layer "F.Cu") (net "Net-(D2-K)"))
 (segment (start 167.9 71.9) (end 169.75 71.9) (width 0.6) (layer "F.Cu") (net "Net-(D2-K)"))
 (segment (start 161.5 63) (end 161.5 69.25) (width 0.6) (layer "F.Cu") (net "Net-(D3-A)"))
 (segment (start 175.5 92) (end 175.5 91.3) (width 0.6) (layer "F.Cu") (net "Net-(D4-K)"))
 (segment (start 175.5 91.3) (end 172.5 88.3) (width 0.6) (layer "F.Cu") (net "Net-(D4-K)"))
 (segment (start 172.5 85.5) (end 174.03 83.97) (width 0.6) (layer "F.Cu") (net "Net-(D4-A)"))
 (segment (start 182.135 86.365) (end 180.9125 86.365) (width 0.6) (layer "F.Cu") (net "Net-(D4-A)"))
 (segment (start 178.2 87.883681) (end 178.2 90.7) (width 0.6) (layer "F.Cu") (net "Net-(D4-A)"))
 (segment (start 182.525 84.529316) (end 182.525 85.975) (width 0.6) (layer "F.Cu") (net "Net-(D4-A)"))
 (segment (start 174.03 83.97) (end 181.965684 83.97) (width 0.6) (layer "F.Cu") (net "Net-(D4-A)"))
 (segment (start 180.9125 86.365) (end 179.718682 86.365) (width 0.6) (layer "F.Cu") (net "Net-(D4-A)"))
 (segment (start 178.2 90.7) (end 179 91.5) (width 0.6) (layer "F.Cu") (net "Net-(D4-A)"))
 (segment (start 179.718682 86.365) (end 178.2 87.883681) (width 0.6) (layer "F.Cu") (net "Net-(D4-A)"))
 (segment (start 179 92.04) (end 184.46 97.5) (width 0.6) (layer "F.Cu") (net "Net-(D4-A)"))
 (segment (start 181.965684 83.97) (end 182.525 84.529316) (width 0.6) (layer "F.Cu") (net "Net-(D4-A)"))
 (segment (start 182.525 85.975) (end 182.135 86.365) (width 0.6) (layer "F.Cu") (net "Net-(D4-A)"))
 (segment (start 179 91.5) (end 179 92.04) (width 0.6) (layer "F.Cu") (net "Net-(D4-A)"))
 (segment (start 190.7 70.5) (end 190.7 74.8) (width 0.6) (layer "F.Cu") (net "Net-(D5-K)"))
 (segment (start 190.7 74.8) (end 190 75.5) (width 0.6) (layer "F.Cu") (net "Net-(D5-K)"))
 (segment (start 179.433046 85.095) (end 177.1 87.428046) (width 0.6) (layer "F.Cu") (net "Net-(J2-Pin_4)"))
 (segment (start 177.1 87.428046) (end 177.1 92.68) (width 0.6) (layer "F.Cu") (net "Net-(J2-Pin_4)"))
 (segment (start 180.9125 85.095) (end 179.433046 85.095) (width 0.6) (layer "F.Cu") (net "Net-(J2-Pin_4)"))
 (segment (start 177.1 92.68) (end 181.92 97.5) (width 0.6) (layer "F.Cu") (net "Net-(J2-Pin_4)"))
 (segment (start 185.647842 83.80084) (end 185.375 84.073682) (width 0.6) (layer "F.Cu") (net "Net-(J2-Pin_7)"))
 (segment (start 186.893681 87.635) (end 188.0875 87.635) (width 0.6) (layer "F.Cu") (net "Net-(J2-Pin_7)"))
 (segment (start 185.647842 83.703476) (end 185.647842 83.80084) (width 0.6) (layer "F.Cu") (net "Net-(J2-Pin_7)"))
 (segment (start 186.475 94.435) (end 189.54 97.5) (width 0.6) (layer "F.Cu") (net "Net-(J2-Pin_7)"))
 (segment (start 171.7 80.9) (end 182.844366 80.9) (width 0.6) (layer "F.Cu") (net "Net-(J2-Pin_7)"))
 (segment (start 188.0875 87.635) (end 187.179316 87.635) (width 0.6) (layer "F.Cu") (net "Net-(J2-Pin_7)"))
 (segment (start 186.475 88.339316) (end 186.475 94.435) (width 0.6) (layer "F.Cu") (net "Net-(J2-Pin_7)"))
 (segment (start 187.179316 87.635) (end 186.475 88.339316) (width 0.6) (layer "F.Cu") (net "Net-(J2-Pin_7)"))
 (segment (start 185.375 86.116319) (end 186.893681 87.635) (width 0.6) (layer "F.Cu") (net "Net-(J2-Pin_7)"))
 (segment (start 168 76.5) (end 168 77.2) (width 0.6) (layer "F.Cu") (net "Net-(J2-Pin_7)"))
 (segment (start 185.375 84.073682) (end 185.375 86.116319) (width 0.6) (layer "F.Cu") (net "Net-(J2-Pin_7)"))
 (segment (start 168 77.2) (end 171.7 80.9) (width 0.6) (layer "F.Cu") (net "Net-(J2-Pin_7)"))
 (segment (start 182.844366 80.9) (end 185.647842 83.703476) (width 0.6) (layer "F.Cu") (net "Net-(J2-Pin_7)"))
 (segment (start 179.3 89.8) (end 187 97.5) (width 0.6) (layer "F.Cu") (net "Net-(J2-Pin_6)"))
 (segment (start 180.9125 87.635) (end 180.004316 87.635) (width 0.6) (layer "F.Cu") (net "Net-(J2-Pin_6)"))
 (segment (start 180.004316 87.635) (end 179.3 88.339316) (width 0.6) (layer "F.Cu") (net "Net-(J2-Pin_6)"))
 (segment (start 179.3 88.339316) (end 179.3 89.8) (width 0.6) (layer "F.Cu") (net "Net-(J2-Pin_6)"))
 (segment (start 194.62 95.4375) (end 194.62 97.5) (width 0.6) (layer "F.Cu") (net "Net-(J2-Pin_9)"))
 (segment (start 188.0875 88.905) (end 194.62 95.4375) (width 0.6) (layer "F.Cu") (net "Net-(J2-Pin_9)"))
 (segment (start 186.475 84.529316) (end 186.475 85.660684) (width 0.6) (layer "F.Cu") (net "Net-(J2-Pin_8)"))
 (segment (start 186.747842 83.247842) (end 186.747842 84.247842) (width 0.6) (layer "F.Cu") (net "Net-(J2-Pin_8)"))
 (segment (start 173 79.5) (end 183 79.5) (width 0.6) (layer "F.Cu") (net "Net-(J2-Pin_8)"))
 (segment (start 197.793453 99.2) (end 193.78 99.2) (width 0.6) (layer "F.Cu") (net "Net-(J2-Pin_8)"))
 (segment (start 193.78 99.2) (end 192.08 97.5) (width 0.6) (layer "F.Cu") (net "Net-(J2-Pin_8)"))
 (segment (start 198.81 98.183453) (end 197.793453 99.2) (width 0.6) (layer "F.Cu") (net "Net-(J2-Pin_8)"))
 (segment (start 186.747842 84.247842) (end 186.752158 84.252158) (width 0.6) (layer "F.Cu") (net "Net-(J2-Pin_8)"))
 (segment (start 186.475 85.660684) (end 187.179316 86.365) (width 0.6) (layer "F.Cu") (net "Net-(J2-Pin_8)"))
 (segment (start 190.865 86.365) (end 198.81 94.31) (width 0.6) (layer "F.Cu") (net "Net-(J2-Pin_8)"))
 (segment (start 198.81 94.31) (end 198.81 98.183453) (width 0.6) (layer "F.Cu") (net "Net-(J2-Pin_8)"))
 (segment (start 188.0875 86.365) (end 190.865 86.365) (width 0.6) (layer "F.Cu") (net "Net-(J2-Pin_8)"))
 (segment (start 186.752158 84.252158) (end 186.475 84.529316) (width 0.6) (layer "F.Cu") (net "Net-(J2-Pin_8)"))
 (segment (start 187.179316 86.365) (end 188.0875 86.365) (width 0.6) (layer "F.Cu") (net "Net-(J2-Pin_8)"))
 (segment (start 183 79.5) (end 186.747842 83.247842) (width 0.6) (layer "F.Cu") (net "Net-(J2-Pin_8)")))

